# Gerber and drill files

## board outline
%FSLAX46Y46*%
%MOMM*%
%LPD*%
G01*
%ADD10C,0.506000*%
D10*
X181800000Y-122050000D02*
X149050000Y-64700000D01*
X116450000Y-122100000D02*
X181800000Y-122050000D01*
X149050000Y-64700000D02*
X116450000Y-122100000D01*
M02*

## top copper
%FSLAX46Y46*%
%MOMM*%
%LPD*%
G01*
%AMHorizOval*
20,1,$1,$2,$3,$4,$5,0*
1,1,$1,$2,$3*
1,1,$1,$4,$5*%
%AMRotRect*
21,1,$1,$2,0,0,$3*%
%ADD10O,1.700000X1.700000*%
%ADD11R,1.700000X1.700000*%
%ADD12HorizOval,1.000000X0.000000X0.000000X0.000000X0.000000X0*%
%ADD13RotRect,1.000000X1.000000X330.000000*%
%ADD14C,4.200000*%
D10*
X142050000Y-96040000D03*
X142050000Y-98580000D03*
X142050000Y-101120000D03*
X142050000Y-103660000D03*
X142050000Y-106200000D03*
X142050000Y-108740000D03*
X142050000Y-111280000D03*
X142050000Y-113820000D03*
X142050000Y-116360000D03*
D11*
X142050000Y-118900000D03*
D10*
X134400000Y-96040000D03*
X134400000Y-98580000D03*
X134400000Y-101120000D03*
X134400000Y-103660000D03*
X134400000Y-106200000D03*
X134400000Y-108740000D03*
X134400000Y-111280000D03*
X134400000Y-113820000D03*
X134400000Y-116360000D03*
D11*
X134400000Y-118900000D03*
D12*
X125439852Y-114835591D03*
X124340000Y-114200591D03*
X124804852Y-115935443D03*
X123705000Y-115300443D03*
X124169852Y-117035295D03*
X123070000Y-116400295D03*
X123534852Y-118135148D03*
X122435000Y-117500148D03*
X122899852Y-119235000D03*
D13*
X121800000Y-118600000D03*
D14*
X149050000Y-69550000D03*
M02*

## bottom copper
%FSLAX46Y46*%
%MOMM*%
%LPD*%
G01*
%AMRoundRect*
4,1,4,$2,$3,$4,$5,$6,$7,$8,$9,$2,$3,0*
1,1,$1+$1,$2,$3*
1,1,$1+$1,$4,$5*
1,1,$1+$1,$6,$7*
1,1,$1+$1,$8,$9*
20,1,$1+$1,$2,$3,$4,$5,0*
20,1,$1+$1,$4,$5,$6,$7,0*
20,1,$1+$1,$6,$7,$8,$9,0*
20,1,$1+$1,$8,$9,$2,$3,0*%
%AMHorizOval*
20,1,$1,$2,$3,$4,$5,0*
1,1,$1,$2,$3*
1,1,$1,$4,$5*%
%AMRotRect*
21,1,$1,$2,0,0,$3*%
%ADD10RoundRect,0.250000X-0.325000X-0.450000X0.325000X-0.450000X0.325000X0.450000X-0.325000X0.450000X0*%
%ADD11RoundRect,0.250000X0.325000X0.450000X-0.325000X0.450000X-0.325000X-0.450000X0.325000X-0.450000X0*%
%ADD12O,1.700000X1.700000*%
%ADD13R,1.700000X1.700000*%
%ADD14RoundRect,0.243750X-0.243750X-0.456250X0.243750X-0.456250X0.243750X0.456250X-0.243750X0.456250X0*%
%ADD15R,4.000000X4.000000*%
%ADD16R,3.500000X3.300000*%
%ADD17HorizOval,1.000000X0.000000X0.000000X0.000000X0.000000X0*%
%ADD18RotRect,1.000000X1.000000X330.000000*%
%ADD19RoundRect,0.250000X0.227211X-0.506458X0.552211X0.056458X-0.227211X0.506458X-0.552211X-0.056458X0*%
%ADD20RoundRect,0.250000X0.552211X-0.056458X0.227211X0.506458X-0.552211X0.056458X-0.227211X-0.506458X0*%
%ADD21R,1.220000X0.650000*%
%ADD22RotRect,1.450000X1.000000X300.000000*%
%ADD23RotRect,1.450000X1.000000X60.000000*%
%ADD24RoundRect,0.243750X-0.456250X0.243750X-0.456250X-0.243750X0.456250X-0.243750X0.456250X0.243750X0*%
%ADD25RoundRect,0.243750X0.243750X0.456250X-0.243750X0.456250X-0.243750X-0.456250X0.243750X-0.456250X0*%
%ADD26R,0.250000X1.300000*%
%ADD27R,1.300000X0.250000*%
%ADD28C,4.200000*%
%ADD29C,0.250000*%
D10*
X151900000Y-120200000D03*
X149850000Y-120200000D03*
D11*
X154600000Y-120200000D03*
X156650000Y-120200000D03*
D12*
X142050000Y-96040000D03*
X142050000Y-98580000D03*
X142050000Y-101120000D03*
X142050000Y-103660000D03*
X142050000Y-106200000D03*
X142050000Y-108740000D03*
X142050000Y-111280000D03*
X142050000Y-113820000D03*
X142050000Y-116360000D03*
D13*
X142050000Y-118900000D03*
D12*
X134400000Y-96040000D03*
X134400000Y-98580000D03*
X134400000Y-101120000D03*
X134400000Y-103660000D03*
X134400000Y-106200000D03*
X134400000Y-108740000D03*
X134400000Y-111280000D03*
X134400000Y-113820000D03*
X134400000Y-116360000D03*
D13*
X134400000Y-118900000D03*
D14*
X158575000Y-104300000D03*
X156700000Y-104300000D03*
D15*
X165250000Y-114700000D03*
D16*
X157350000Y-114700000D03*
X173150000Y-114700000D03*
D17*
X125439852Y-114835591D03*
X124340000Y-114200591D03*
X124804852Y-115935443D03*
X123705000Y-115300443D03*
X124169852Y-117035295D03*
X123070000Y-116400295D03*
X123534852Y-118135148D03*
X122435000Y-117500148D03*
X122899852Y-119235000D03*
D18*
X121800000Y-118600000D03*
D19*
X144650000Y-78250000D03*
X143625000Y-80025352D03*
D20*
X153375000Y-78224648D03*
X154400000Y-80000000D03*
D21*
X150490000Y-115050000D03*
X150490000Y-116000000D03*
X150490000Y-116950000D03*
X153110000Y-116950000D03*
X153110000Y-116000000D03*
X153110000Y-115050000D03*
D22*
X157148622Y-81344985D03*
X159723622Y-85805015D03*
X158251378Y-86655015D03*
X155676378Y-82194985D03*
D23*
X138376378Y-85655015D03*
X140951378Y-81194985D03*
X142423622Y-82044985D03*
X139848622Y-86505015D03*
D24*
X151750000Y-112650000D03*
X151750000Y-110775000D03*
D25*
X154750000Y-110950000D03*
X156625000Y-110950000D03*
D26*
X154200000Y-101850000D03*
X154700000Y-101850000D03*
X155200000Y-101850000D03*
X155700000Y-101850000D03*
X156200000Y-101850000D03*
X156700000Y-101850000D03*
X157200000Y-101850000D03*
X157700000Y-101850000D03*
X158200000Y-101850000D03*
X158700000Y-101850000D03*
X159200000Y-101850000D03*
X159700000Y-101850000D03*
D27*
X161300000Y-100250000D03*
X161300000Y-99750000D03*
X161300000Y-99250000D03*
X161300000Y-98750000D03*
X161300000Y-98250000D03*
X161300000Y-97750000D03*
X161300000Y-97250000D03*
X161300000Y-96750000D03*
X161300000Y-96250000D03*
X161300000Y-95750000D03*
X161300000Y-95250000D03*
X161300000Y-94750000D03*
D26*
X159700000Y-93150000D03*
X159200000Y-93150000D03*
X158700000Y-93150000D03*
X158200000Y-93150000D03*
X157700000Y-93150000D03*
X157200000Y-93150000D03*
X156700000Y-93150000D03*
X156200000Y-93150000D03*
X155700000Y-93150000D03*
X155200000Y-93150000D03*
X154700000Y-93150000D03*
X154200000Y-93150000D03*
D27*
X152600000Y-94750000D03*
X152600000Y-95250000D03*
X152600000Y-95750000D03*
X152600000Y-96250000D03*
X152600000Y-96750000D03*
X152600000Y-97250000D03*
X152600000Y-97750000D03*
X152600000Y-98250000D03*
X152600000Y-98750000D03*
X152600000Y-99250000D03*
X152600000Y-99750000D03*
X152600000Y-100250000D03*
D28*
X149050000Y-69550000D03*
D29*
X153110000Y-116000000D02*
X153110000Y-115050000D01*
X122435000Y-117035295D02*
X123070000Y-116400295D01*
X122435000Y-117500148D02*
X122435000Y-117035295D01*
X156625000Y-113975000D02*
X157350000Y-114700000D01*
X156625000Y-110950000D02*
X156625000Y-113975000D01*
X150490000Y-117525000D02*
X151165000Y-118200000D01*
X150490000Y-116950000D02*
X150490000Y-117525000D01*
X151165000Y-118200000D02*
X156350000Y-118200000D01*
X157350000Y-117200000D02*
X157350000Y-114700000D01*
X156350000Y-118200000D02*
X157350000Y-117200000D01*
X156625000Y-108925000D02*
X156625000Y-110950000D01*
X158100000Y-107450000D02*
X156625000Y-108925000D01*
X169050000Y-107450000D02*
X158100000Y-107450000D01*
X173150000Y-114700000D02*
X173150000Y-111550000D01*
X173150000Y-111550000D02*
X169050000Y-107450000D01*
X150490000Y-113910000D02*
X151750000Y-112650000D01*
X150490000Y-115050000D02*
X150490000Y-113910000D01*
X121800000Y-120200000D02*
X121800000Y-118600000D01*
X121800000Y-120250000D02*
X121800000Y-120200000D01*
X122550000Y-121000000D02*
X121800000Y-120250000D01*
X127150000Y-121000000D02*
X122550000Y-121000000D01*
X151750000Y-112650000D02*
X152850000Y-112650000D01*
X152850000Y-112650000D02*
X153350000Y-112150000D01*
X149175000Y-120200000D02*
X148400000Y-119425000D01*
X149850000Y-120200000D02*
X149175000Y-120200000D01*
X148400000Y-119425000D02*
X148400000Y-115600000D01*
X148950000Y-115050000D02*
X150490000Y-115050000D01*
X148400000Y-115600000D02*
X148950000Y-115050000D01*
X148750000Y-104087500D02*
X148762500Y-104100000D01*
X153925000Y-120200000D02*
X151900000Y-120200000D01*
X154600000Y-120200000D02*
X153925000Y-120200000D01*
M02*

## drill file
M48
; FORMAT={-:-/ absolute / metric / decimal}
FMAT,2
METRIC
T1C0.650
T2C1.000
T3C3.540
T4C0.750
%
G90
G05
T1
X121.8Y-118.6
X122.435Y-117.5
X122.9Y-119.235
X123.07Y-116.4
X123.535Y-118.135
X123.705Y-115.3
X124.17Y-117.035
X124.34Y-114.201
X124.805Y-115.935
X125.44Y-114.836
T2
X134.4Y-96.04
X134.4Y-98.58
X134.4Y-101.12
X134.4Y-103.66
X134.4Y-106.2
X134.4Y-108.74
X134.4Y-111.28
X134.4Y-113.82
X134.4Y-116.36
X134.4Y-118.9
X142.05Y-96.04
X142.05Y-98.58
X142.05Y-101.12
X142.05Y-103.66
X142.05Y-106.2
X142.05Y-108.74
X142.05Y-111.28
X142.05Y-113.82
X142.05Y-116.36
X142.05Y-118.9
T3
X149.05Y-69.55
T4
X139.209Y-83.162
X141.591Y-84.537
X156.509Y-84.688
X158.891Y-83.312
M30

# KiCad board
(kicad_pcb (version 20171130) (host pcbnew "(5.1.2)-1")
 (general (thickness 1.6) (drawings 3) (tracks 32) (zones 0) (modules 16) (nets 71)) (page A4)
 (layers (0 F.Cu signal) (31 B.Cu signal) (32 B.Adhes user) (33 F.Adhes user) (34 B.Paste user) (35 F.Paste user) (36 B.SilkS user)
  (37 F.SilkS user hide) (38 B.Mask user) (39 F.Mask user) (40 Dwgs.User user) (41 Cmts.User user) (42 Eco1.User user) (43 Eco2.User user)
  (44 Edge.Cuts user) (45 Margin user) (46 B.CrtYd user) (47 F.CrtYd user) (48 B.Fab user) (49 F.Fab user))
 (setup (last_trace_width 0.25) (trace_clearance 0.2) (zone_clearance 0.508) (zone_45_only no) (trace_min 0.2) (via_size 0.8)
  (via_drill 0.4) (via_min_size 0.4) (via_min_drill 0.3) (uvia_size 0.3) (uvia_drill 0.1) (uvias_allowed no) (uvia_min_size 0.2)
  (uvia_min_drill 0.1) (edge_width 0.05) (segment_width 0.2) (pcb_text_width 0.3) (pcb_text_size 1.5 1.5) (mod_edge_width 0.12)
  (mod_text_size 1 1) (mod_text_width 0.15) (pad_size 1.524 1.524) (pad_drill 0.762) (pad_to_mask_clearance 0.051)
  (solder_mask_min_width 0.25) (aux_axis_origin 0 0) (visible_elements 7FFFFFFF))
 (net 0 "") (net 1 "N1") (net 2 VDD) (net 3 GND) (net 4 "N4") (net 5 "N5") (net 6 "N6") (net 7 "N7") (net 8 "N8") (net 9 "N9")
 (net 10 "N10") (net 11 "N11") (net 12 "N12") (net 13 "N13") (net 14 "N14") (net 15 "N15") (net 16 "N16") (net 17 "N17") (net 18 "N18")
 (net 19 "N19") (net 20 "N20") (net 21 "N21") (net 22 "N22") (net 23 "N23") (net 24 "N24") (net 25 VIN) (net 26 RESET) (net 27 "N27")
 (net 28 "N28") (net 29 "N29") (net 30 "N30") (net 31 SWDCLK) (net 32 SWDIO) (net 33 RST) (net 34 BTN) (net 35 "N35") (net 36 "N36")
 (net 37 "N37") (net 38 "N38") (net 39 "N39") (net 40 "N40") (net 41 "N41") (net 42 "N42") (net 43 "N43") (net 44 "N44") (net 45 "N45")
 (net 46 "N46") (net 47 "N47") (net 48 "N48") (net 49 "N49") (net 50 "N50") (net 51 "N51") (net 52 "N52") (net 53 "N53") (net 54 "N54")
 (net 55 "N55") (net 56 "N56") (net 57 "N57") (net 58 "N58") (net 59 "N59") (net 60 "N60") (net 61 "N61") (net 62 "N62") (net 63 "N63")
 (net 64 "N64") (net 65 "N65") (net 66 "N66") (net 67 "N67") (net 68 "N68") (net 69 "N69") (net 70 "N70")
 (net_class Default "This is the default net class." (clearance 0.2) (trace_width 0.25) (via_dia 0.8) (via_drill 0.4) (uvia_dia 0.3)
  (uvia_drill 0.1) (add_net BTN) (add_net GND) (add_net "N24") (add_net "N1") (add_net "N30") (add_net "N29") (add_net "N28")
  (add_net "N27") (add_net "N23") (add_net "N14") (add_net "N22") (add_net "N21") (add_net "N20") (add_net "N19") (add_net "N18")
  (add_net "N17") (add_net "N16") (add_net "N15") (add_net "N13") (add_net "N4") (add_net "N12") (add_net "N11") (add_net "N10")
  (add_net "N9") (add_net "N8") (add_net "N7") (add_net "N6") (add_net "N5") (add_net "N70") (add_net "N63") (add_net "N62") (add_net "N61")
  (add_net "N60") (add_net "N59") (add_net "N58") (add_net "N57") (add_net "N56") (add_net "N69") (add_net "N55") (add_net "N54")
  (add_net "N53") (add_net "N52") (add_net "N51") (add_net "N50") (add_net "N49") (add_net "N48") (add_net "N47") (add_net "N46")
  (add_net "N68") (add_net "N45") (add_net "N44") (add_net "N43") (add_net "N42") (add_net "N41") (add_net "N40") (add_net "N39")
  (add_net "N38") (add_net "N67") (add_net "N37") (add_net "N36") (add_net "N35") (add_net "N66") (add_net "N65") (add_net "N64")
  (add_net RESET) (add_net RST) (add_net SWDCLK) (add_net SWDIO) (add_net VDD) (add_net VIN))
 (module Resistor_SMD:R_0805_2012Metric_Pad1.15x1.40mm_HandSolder (layer B.Cu) (at 150.875 120.2)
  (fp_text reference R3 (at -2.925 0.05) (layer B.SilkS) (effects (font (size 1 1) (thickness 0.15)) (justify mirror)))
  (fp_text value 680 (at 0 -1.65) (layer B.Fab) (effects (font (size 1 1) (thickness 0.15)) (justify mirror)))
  (pad 2 smd roundrect (at 1.025 0) (size 1.15 1.4) (layers B.Cu B.Paste B.Mask) (roundrect_rratio 0.217391) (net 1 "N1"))
  (pad 1 smd roundrect (at -1.025 0) (size 1.15 1.4) (layers B.Cu B.Paste B.Mask) (roundrect_rratio 0.217391) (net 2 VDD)))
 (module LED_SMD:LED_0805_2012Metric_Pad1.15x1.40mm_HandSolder (layer B.Cu) (at 155.625 120.2 180)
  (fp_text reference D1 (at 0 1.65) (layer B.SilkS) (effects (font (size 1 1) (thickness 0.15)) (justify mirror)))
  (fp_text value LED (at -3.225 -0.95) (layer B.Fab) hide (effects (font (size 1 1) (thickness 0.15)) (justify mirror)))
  (pad 2 smd roundrect (at 1.025 0 180) (size 1.15 1.4) (layers B.Cu B.Paste B.Mask) (roundrect_rratio 0.217391) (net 1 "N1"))
  (pad 1 smd roundrect (at -1.025 0 180) (size 1.15 1.4) (layers B.Cu B.Paste B.Mask) (roundrect_rratio 0.217391) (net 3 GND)))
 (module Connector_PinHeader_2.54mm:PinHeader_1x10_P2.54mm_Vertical (layer B.Cu) (at 142.05 118.9)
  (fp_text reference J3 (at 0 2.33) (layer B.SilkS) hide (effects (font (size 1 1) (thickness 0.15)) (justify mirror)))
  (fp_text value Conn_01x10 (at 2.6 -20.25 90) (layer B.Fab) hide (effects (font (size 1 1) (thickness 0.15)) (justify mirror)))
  (pad 10 thru_hole oval (at 0 -22.86) (size 1.7 1.7) (drill 1) (layers *.Cu *.Mask) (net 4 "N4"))
  (pad 9 thru_hole oval (at 0 -20.32) (size 1.7 1.7) (drill 1) (layers *.Cu *.Mask) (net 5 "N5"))
  (pad 8 thru_hole oval (at 0 -17.78) (size 1.7 1.7) (drill 1) (layers *.Cu *.Mask) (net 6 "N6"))
  (pad 7 thru_hole oval (at 0 -15.24) (size 1.7 1.7) (drill 1) (layers *.Cu *.Mask) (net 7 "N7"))
  (pad 6 thru_hole oval (at 0 -12.7) (size 1.7 1.7) (drill 1) (layers *.Cu *.Mask) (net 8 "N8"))
  (pad 5 thru_hole oval (at 0 -10.16) (size 1.7 1.7) (drill 1) (layers *.Cu *.Mask) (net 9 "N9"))
  (pad 4 thru_hole oval (at 0 -7.62) (size 1.7 1.7) (drill 1) (layers *.Cu *.Mask) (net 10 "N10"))
  (pad 3 thru_hole oval (at 0 -5.08) (size 1.7 1.7) (drill 1) (layers *.Cu *.Mask) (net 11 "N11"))
  (pad 2 thru_hole oval (at 0 -2.54) (size 1.7 1.7) (drill 1) (layers *.Cu *.Mask) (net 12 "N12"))
  (pad 1 thru_hole rect (at 0 0) (size 1.7 1.7) (drill 1) (layers *.Cu *.Mask) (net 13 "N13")))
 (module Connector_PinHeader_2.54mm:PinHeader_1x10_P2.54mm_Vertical (layer B.Cu) (at 134.4 118.9)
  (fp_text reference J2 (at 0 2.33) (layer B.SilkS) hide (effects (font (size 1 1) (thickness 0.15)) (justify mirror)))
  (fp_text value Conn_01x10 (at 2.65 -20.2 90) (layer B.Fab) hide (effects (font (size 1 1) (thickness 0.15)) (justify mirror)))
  (pad 10 thru_hole oval (at 0 -22.86) (size 1.7 1.7) (drill 1) (layers *.Cu *.Mask) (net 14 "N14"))
  (pad 9 thru_hole oval (at 0 -20.32) (size 1.7 1.7) (drill 1) (layers *.Cu *.Mask) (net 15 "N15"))
  (pad 8 thru_hole oval (at 0 -17.78) (size 1.7 1.7) (drill 1) (layers *.Cu *.Mask) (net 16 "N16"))
  (pad 7 thru_hole oval (at 0 -15.24) (size 1.7 1.7) (drill 1) (layers *.Cu *.Mask) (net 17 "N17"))
  (pad 6 thru_hole oval (at 0 -12.7) (size 1.7 1.7) (drill 1) (layers *.Cu *.Mask) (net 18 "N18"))
  (pad 5 thru_hole oval (at 0 -10.16) (size 1.7 1.7) (drill 1) (layers *.Cu *.Mask) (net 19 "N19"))
  (pad 4 thru_hole oval (at 0 -7.62) (size 1.7 1.7) (drill 1) (layers *.Cu *.Mask) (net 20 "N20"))
  (pad 3 thru_hole oval (at 0 -5.08) (size 1.7 1.7) (drill 1) (layers *.Cu *.Mask) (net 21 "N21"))
  (pad 2 thru_hole oval (at 0 -2.54) (size 1.7 1.7) (drill 1) (layers *.Cu *.Mask) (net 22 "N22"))
  (pad 1 thru_hole rect (at 0 0) (size 1.7 1.7) (drill 1) (layers *.Cu *.Mask) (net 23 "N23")))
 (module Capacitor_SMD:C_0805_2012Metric (layer B.Cu) (at 157.6375 104.3)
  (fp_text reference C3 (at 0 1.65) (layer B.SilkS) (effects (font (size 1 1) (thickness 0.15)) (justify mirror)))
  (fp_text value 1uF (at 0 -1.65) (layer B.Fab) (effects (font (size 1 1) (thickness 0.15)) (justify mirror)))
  (pad 2 smd roundrect (at 0.9375 0) (size 0.975 1.4) (layers B.Cu B.Paste B.Mask) (roundrect_rratio 0.25) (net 3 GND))
  (pad 1 smd roundrect (at -0.9375 0) (size 0.975 1.4) (layers B.Cu B.Paste B.Mask) (roundrect_rratio 0.25) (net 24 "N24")))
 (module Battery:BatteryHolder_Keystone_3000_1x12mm (layer B.Cu) (at 165.25 114.7 180)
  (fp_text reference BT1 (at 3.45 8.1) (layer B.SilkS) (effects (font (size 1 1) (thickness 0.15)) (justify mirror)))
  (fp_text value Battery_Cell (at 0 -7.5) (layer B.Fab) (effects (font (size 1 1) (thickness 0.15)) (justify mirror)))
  (pad 2 smd rect (at 0 0 180) (size 4 4) (layers B.Cu B.Mask) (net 3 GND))
  (pad 1 smd rect (at 7.9 0 180) (size 3.5 3.3) (layers B.Cu B.Paste B.Mask) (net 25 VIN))
  (pad 1 smd rect (at -7.9 0 180) (size 3.5 3.3) (layers B.Cu B.Paste B.Mask) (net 25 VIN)))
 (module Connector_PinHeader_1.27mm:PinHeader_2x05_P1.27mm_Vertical (layer B.Cu) (at 121.8 118.6 330)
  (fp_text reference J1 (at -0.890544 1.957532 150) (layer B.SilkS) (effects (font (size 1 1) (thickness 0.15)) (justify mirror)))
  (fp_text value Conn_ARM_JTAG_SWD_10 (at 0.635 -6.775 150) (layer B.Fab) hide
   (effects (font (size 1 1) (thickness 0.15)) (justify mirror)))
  (pad 10 thru_hole oval (at 1.27 -5.08 330) (size 1 1) (drill 0.65) (layers *.Cu *.Mask) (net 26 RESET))
  (pad 9 thru_hole oval (at 0 -5.08 330) (size 1 1) (drill 0.65) (layers *.Cu *.Mask) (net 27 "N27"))
  (pad 8 thru_hole oval (at 1.27 -3.81 330) (size 1 1) (drill 0.65) (layers *.Cu *.Mask) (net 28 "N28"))
  (pad 7 thru_hole oval (at 0 -3.81 330) (size 1 1) (drill 0.65) (layers *.Cu *.Mask) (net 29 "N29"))
  (pad 6 thru_hole oval (at 1.27 -2.54 330) (size 1 1) (drill 0.65) (layers *.Cu *.Mask) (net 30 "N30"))
  (pad 5 thru_hole oval (at 0 -2.54 330) (size 1 1) (drill 0.65) (layers *.Cu *.Mask) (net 3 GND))
  (pad 4 thru_hole oval (at 1.27 -1.27 330) (size 1 1) (drill 0.65) (layers *.Cu *.Mask) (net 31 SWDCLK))
  (pad 3 thru_hole oval (at 0 -1.27 330) (size 1 1) (drill 0.65) (layers *.Cu *.Mask) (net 3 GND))
  (pad 2 thru_hole oval (at 1.27 0 330) (size 1 1) (drill 0.65) (layers *.Cu *.Mask) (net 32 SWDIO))
  (pad 1 thru_hole rect (at 0 0 330) (size 1 1) (drill 0.65) (layers *.Cu *.Mask) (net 2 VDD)))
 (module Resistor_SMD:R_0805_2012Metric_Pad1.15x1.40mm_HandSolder (layer B.Cu) (at 144.1375 79.137676 60)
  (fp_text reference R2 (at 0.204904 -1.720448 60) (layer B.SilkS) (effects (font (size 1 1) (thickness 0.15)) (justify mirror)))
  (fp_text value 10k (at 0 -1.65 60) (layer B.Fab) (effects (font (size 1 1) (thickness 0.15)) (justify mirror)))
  (pad 2 smd roundrect (at 1.025 0 60) (size 1.15 1.4) (layers B.Cu B.Paste B.Mask) (roundrect_rratio 0.217391) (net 2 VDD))
  (pad 1 smd roundrect (at -1.025 0 60) (size 1.15 1.4) (layers B.Cu B.Paste B.Mask) (roundrect_rratio 0.217391) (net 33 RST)))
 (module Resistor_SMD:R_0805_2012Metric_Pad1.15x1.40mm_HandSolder (layer B.Cu) (at 153.8875 79.112324 120)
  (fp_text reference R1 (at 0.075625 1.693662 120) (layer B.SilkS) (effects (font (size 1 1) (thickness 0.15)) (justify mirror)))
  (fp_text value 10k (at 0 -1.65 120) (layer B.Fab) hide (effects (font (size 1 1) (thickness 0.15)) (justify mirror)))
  (pad 2 smd roundrect (at 1.025 0 120) (size 1.15 1.4) (layers B.Cu B.Paste B.Mask) (roundrect_rratio 0.217391) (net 3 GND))
  (pad 1 smd roundrect (at -1.025 0 120) (size 1.15 1.4) (layers B.Cu B.Paste B.Mask) (roundrect_rratio 0.217391) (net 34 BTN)))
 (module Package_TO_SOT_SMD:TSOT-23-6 (layer B.Cu) (at 151.8 116 180)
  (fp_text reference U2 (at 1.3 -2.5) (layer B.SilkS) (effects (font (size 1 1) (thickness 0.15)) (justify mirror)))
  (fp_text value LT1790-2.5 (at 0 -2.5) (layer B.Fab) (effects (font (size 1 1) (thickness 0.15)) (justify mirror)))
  (pad 6 smd rect (at 1.31 0.95 180) (size 1.22 0.65) (layers B.Cu B.Paste B.Mask) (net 2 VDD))
  (pad 5 smd rect (at 1.31 0 180) (size 1.22 0.65) (layers B.Cu B.Paste B.Mask))
  (pad 4 smd rect (at 1.31 -0.95 180) (size 1.22 0.65) (layers B.Cu B.Paste B.Mask) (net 25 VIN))
  (pad 3 smd rect (at -1.31 -0.95 180) (size 1.22 0.65) (layers B.Cu B.Paste B.Mask))
  (pad 2 smd rect (at -1.31 0 180) (size 1.22 0.65) (layers B.Cu B.Paste B.Mask) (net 3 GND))
  (pad 1 smd rect (at -1.31 0.95 180) (size 1.22 0.65) (layers B.Cu B.Paste B.Mask) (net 3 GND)))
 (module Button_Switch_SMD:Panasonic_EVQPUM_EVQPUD (layer B.Cu) (at 157.7 84 120)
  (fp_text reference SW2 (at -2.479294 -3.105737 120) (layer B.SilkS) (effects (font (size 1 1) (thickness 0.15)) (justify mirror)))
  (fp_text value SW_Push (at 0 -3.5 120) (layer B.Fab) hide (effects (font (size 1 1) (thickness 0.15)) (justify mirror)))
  (pad "" np_thru_hole circle (at 0 1.375 300) (size 0.75 0.75) (drill 0.75) (layers *.Cu *.Mask))
  (pad "" np_thru_hole circle (at 0 -1.375 300) (size 0.75 0.75) (drill 0.75) (layers *.Cu *.Mask))
  (pad 1 smd rect (at 2.575 0.85 300) (size 1.45 1) (layers B.Cu B.Paste B.Mask) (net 2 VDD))
  (pad 1 smd rect (at -2.575 0.85 300) (size 1.45 1) (layers B.Cu B.Paste B.Mask) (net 2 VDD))
  (pad 2 smd rect (at -2.575 -0.85 300) (size 1.45 1) (layers B.Cu B.Paste B.Mask) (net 34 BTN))
  (pad 2 smd rect (at 2.575 -0.85 300) (size 1.45 1) (layers B.Cu B.Paste B.Mask) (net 34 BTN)))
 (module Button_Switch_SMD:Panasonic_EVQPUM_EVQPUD (layer B.Cu) (at 140.4 83.85 240)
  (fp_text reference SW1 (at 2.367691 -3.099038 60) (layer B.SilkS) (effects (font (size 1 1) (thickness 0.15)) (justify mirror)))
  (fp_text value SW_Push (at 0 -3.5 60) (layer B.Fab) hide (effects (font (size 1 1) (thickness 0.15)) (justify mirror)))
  (pad "" np_thru_hole circle (at 0 1.375 60) (size 0.75 0.75) (drill 0.75) (layers *.Cu *.Mask))
  (pad "" np_thru_hole circle (at 0 -1.375 60) (size 0.75 0.75) (drill 0.75) (layers *.Cu *.Mask))
  (pad 1 smd rect (at 2.575 0.85 60) (size 1.45 1) (layers B.Cu B.Paste B.Mask) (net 3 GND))
  (pad 1 smd rect (at -2.575 0.85 60) (size 1.45 1) (layers B.Cu B.Paste B.Mask) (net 3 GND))
  (pad 2 smd rect (at -2.575 -0.85 60) (size 1.45 1) (layers B.Cu B.Paste B.Mask) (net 33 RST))
  (pad 2 smd rect (at 2.575 -0.85 60) (size 1.45 1) (layers B.Cu B.Paste B.Mask) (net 33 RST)))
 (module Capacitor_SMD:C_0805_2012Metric (layer B.Cu) (at 151.75 111.7125 270)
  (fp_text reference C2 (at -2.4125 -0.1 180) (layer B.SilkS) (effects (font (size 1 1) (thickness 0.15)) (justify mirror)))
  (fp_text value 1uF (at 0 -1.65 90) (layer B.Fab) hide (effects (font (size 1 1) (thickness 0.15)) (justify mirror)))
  (pad 2 smd roundrect (at 0.9375 0 270) (size 0.975 1.4) (layers B.Cu B.Paste B.Mask) (roundrect_rratio 0.25) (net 2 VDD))
  (pad 1 smd roundrect (at -0.9375 0 270) (size 0.975 1.4) (layers B.Cu B.Paste B.Mask) (roundrect_rratio 0.25) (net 3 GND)))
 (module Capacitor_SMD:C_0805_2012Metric (layer B.Cu) (at 155.6875 110.95 180)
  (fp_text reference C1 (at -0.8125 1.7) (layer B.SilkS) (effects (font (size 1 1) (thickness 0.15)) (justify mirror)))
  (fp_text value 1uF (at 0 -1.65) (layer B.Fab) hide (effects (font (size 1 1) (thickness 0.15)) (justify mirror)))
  (pad 2 smd roundrect (at 0.9375 0 180) (size 0.975 1.4) (layers B.Cu B.Paste B.Mask) (roundrect_rratio 0.25) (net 3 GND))
  (pad 1 smd roundrect (at -0.9375 0 180) (size 0.975 1.4) (layers B.Cu B.Paste B.Mask) (roundrect_rratio 0.25) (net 25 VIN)))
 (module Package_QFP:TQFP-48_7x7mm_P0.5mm (layer B.Cu) (at 156.95 97.5)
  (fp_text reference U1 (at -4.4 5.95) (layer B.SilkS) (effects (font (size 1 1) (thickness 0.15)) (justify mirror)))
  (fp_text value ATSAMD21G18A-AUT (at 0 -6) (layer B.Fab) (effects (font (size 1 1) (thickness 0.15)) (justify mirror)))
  (pad 48 smd rect (at -2.75 4.35 270) (size 1.3 0.25) (layers B.Cu B.Paste B.Mask) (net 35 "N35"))
  (pad 47 smd rect (at -2.25 4.35 270) (size 1.3 0.25) (layers B.Cu B.Paste B.Mask) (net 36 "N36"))
  (pad 46 smd rect (at -1.75 4.35 270) (size 1.3 0.25) (layers B.Cu B.Paste B.Mask) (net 32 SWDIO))
  (pad 45 smd rect (at -1.25 4.35 270) (size 1.3 0.25) (layers B.Cu B.Paste B.Mask) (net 31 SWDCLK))
  (pad 44 smd rect (at -0.75 4.35 270) (size 1.3 0.25) (layers B.Cu B.Paste B.Mask) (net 2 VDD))
  (pad 43 smd rect (at -0.25 4.35 270) (size 1.3 0.25) (layers B.Cu B.Paste B.Mask) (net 24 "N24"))
  (pad 42 smd rect (at 0.25 4.35 270) (size 1.3 0.25) (layers B.Cu B.Paste B.Mask) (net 3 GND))
  (pad 41 smd rect (at 0.75 4.35 270) (size 1.3 0.25) (layers B.Cu B.Paste B.Mask) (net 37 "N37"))
  (pad 40 smd rect (at 1.25 4.35 270) (size 1.3 0.25) (layers B.Cu B.Paste B.Mask) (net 26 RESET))
  (pad 39 smd rect (at 1.75 4.35 270) (size 1.3 0.25) (layers B.Cu B.Paste B.Mask) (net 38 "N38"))
  (pad 38 smd rect (at 2.25 4.35 270) (size 1.3 0.25) (layers B.Cu B.Paste B.Mask) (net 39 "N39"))
  (pad 37 smd rect (at 2.75 4.35 270) (size 1.3 0.25) (layers B.Cu B.Paste B.Mask) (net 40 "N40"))
  (pad 36 smd rect (at 4.35 2.75) (size 1.3 0.25) (layers B.Cu B.Paste B.Mask) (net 2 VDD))
  (pad 35 smd rect (at 4.35 2.25) (size 1.3 0.25) (layers B.Cu B.Paste B.Mask) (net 3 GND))
  (pad 34 smd rect (at 4.35 1.75) (size 1.3 0.25) (layers B.Cu B.Paste B.Mask) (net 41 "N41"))
  (pad 33 smd rect (at 4.35 1.25) (size 1.3 0.25) (layers B.Cu B.Paste B.Mask) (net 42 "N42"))
  (pad 32 smd rect (at 4.35 0.75) (size 1.3 0.25) (layers B.Cu B.Paste B.Mask) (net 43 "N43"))
  (pad 31 smd rect (at 4.35 0.25) (size 1.3 0.25) (layers B.Cu B.Paste B.Mask) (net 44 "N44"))
  (pad 30 smd rect (at 4.35 -0.25) (size 1.3 0.25) (layers B.Cu B.Paste B.Mask) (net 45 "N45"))
  (pad 29 smd rect (at 4.35 -0.75) (size 1.3 0.25) (layers B.Cu B.Paste B.Mask) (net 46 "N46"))
  (pad 28 smd rect (at 4.35 -1.25) (size 1.3 0.25) (layers B.Cu B.Paste B.Mask) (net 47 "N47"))
  (pad 27 smd rect (at 4.35 -1.75) (size 1.3 0.25) (layers B.Cu B.Paste B.Mask) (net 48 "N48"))
  (pad 26 smd rect (at 4.35 -2.25) (size 1.3 0.25) (layers B.Cu B.Paste B.Mask) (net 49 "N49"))
  (pad 25 smd rect (at 4.35 -2.75) (size 1.3 0.25) (layers B.Cu B.Paste B.Mask) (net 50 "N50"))
  (pad 24 smd rect (at 2.75 -4.35 270) (size 1.3 0.25) (layers B.Cu B.Paste B.Mask) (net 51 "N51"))
  (pad 23 smd rect (at 2.25 -4.35 270) (size 1.3 0.25) (layers B.Cu B.Paste B.Mask) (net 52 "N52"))
  (pad 22 smd rect (at 1.75 -4.35 270) (size 1.3 0.25) (layers B.Cu B.Paste B.Mask) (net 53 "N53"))
  (pad 21 smd rect (at 1.25 -4.35 270) (size 1.3 0.25) (layers B.Cu B.Paste B.Mask) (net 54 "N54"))
  (pad 20 smd rect (at 0.75 -4.35 270) (size 1.3 0.25) (layers B.Cu B.Paste B.Mask) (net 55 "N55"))
  (pad 19 smd rect (at 0.25 -4.35 270) (size 1.3 0.25) (layers B.Cu B.Paste B.Mask) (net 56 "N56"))
  (pad 18 smd rect (at -0.25 -4.35 270) (size 1.3 0.25) (layers B.Cu B.Paste B.Mask) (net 3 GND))
  (pad 17 smd rect (at -0.75 -4.35 270) (size 1.3 0.25) (layers B.Cu B.Paste B.Mask) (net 2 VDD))
  (pad 16 smd rect (at -1.25 -4.35 270) (size 1.3 0.25) (layers B.Cu B.Paste B.Mask) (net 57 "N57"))
  (pad 15 smd rect (at -1.75 -4.35 270) (size 1.3 0.25) (layers B.Cu B.Paste B.Mask) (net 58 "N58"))
  (pad 14 smd rect (at -2.25 -4.35 270) (size 1.3 0.25) (layers B.Cu B.Paste B.Mask) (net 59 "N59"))
  (pad 13 smd rect (at -2.75 -4.35 270) (size 1.3 0.25) (layers B.Cu B.Paste B.Mask) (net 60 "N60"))
  (pad 12 smd rect (at -4.35 -2.75) (size 1.3 0.25) (layers B.Cu B.Paste B.Mask) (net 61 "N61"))
  (pad 11 smd rect (at -4.35 -2.25) (size 1.3 0.25) (layers B.Cu B.Paste B.Mask) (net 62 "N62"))
  (pad 10 smd rect (at -4.35 -1.75) (size 1.3 0.25) (layers B.Cu B.Paste B.Mask) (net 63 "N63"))
  (pad 9 smd rect (at -4.35 -1.25) (size 1.3 0.25) (layers B.Cu B.Paste B.Mask) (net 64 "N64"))
  (pad 8 smd rect (at -4.35 -0.75) (size 1.3 0.25) (layers B.Cu B.Paste B.Mask) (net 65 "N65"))
  (pad 7 smd rect (at -4.35 -0.25) (size 1.3 0.25) (layers B.Cu B.Paste B.Mask) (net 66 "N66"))
  (pad 6 smd rect (at -4.35 0.25) (size 1.3 0.25) (layers B.Cu B.Paste B.Mask) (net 2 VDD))
  (pad 5 smd rect (at -4.35 0.75) (size 1.3 0.25) (layers B.Cu B.Paste B.Mask) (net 3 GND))
  (pad 4 smd rect (at -4.35 1.25) (size 1.3 0.25) (layers B.Cu B.Paste B.Mask) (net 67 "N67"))
  (pad 3 smd rect (at -4.35 1.75) (size 1.3 0.25) (layers B.Cu B.Paste B.Mask) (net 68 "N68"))
  (pad 2 smd rect (at -4.35 2.25) (size 1.3 0.25) (layers B.Cu B.Paste B.Mask) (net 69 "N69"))
  (pad 1 smd rect (at -4.35 2.75) (size 1.3 0.25) (layers B.Cu B.Paste B.Mask) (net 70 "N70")))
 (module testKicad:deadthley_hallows (layer F.Cu) (at 148.59 93.98)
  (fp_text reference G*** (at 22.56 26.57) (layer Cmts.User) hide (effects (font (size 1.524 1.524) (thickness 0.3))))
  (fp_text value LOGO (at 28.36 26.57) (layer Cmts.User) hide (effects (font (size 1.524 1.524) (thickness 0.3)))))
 (gr_line (start 181.8 122.05) (end 149.05 64.7) (layer Edge.Cuts) (width 0.506))
 (gr_line (start 116.45 122.1) (end 181.8 122.05) (layer Edge.Cuts) (width 0.506))
 (gr_line (start 149.05 64.7) (end 116.45 122.1) (layer Edge.Cuts) (width 0.506))
 (via (at 149.05 69.55) (size 4.2) (drill 3.54) (layers F.Cu B.Cu) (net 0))
 (segment (start 153.11 116) (end 153.11 115.05) (width 0.25) (layer B.Cu) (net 3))
 (segment (start 122.435 117.035295) (end 123.07 116.400295) (width 0.25) (layer B.Cu) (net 3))
 (segment (start 122.435 117.500148) (end 122.435 117.035295) (width 0.25) (layer B.Cu) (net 3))
 (segment (start 156.625 113.975) (end 157.35 114.7) (width 0.25) (layer B.Cu) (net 25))
 (segment (start 156.625 110.95) (end 156.625 113.975) (width 0.25) (layer B.Cu) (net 25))
 (segment (start 150.49 117.525) (end 151.165 118.2) (width 0.25) (layer B.Cu) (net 25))
 (segment (start 150.49 116.95) (end 150.49 117.525) (width 0.25) (layer B.Cu) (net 25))
 (segment (start 151.165 118.2) (end 156.35 118.2) (width 0.25) (layer B.Cu) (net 25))
 (segment (start 157.35 117.2) (end 157.35 114.7) (width 0.25) (layer B.Cu) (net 25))
 (segment (start 156.35 118.2) (end 157.35 117.2) (width 0.25) (layer B.Cu) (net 25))
 (segment (start 156.625 108.925) (end 156.625 110.95) (width 0.25) (layer B.Cu) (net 25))
 (segment (start 158.1 107.45) (end 156.625 108.925) (width 0.25) (layer B.Cu) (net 25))
 (segment (start 169.05 107.45) (end 158.1 107.45) (width 0.25) (layer B.Cu) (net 25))
 (segment (start 173.15 114.7) (end 173.15 111.55) (width 0.25) (layer B.Cu) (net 25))
 (segment (start 173.15 111.55) (end 169.05 107.45) (width 0.25) (layer B.Cu) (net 25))
 (segment (start 150.49 113.91) (end 151.75 112.65) (width 0.25) (layer B.Cu) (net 2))
 (segment (start 150.49 115.05) (end 150.49 113.91) (width 0.25) (layer B.Cu) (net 2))
 (segment (start 121.8 120.2) (end 121.8 118.6) (width 0.25) (layer B.Cu) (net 2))
 (segment (start 121.8 120.25) (end 121.8 120.2) (width 0.25) (layer B.Cu) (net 2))
 (segment (start 122.55 121) (end 121.8 120.25) (width 0.25) (layer B.Cu) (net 2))
 (segment (start 127.15 121) (end 122.55 121) (width 0.25) (layer B.Cu) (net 2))
 (segment (start 151.75 112.65) (end 152.85 112.65) (width 0.25) (layer B.Cu) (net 2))
 (segment (start 152.85 112.65) (end 153.35 112.15) (width 0.25) (layer B.Cu) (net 2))
 (segment (start 149.175 120.2) (end 148.4 119.425) (width 0.25) (layer B.Cu) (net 2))
 (segment (start 149.85 120.2) (end 149.175 120.2) (width 0.25) (layer B.Cu) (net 2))
 (segment (start 148.4 119.425) (end 148.4 115.6) (width 0.25) (layer B.Cu) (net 2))
 (segment (start 148.95 115.05) (end 150.49 115.05) (width 0.25) (layer B.Cu) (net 2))
 (segment (start 148.4 115.6) (end 148.95 115.05) (width 0.25) (layer B.Cu) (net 2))
 (segment (start 148.75 104.0875) (end 148.7625 104.1) (width 0.25) (layer B.Cu) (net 24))
 (segment (start 153.925 120.2) (end 151.9 120.2) (width 0.25) (layer B.Cu) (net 1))
 (segment (start 154.6 120.2) (end 153.925 120.2) (width 0.25) (layer B.Cu) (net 1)))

